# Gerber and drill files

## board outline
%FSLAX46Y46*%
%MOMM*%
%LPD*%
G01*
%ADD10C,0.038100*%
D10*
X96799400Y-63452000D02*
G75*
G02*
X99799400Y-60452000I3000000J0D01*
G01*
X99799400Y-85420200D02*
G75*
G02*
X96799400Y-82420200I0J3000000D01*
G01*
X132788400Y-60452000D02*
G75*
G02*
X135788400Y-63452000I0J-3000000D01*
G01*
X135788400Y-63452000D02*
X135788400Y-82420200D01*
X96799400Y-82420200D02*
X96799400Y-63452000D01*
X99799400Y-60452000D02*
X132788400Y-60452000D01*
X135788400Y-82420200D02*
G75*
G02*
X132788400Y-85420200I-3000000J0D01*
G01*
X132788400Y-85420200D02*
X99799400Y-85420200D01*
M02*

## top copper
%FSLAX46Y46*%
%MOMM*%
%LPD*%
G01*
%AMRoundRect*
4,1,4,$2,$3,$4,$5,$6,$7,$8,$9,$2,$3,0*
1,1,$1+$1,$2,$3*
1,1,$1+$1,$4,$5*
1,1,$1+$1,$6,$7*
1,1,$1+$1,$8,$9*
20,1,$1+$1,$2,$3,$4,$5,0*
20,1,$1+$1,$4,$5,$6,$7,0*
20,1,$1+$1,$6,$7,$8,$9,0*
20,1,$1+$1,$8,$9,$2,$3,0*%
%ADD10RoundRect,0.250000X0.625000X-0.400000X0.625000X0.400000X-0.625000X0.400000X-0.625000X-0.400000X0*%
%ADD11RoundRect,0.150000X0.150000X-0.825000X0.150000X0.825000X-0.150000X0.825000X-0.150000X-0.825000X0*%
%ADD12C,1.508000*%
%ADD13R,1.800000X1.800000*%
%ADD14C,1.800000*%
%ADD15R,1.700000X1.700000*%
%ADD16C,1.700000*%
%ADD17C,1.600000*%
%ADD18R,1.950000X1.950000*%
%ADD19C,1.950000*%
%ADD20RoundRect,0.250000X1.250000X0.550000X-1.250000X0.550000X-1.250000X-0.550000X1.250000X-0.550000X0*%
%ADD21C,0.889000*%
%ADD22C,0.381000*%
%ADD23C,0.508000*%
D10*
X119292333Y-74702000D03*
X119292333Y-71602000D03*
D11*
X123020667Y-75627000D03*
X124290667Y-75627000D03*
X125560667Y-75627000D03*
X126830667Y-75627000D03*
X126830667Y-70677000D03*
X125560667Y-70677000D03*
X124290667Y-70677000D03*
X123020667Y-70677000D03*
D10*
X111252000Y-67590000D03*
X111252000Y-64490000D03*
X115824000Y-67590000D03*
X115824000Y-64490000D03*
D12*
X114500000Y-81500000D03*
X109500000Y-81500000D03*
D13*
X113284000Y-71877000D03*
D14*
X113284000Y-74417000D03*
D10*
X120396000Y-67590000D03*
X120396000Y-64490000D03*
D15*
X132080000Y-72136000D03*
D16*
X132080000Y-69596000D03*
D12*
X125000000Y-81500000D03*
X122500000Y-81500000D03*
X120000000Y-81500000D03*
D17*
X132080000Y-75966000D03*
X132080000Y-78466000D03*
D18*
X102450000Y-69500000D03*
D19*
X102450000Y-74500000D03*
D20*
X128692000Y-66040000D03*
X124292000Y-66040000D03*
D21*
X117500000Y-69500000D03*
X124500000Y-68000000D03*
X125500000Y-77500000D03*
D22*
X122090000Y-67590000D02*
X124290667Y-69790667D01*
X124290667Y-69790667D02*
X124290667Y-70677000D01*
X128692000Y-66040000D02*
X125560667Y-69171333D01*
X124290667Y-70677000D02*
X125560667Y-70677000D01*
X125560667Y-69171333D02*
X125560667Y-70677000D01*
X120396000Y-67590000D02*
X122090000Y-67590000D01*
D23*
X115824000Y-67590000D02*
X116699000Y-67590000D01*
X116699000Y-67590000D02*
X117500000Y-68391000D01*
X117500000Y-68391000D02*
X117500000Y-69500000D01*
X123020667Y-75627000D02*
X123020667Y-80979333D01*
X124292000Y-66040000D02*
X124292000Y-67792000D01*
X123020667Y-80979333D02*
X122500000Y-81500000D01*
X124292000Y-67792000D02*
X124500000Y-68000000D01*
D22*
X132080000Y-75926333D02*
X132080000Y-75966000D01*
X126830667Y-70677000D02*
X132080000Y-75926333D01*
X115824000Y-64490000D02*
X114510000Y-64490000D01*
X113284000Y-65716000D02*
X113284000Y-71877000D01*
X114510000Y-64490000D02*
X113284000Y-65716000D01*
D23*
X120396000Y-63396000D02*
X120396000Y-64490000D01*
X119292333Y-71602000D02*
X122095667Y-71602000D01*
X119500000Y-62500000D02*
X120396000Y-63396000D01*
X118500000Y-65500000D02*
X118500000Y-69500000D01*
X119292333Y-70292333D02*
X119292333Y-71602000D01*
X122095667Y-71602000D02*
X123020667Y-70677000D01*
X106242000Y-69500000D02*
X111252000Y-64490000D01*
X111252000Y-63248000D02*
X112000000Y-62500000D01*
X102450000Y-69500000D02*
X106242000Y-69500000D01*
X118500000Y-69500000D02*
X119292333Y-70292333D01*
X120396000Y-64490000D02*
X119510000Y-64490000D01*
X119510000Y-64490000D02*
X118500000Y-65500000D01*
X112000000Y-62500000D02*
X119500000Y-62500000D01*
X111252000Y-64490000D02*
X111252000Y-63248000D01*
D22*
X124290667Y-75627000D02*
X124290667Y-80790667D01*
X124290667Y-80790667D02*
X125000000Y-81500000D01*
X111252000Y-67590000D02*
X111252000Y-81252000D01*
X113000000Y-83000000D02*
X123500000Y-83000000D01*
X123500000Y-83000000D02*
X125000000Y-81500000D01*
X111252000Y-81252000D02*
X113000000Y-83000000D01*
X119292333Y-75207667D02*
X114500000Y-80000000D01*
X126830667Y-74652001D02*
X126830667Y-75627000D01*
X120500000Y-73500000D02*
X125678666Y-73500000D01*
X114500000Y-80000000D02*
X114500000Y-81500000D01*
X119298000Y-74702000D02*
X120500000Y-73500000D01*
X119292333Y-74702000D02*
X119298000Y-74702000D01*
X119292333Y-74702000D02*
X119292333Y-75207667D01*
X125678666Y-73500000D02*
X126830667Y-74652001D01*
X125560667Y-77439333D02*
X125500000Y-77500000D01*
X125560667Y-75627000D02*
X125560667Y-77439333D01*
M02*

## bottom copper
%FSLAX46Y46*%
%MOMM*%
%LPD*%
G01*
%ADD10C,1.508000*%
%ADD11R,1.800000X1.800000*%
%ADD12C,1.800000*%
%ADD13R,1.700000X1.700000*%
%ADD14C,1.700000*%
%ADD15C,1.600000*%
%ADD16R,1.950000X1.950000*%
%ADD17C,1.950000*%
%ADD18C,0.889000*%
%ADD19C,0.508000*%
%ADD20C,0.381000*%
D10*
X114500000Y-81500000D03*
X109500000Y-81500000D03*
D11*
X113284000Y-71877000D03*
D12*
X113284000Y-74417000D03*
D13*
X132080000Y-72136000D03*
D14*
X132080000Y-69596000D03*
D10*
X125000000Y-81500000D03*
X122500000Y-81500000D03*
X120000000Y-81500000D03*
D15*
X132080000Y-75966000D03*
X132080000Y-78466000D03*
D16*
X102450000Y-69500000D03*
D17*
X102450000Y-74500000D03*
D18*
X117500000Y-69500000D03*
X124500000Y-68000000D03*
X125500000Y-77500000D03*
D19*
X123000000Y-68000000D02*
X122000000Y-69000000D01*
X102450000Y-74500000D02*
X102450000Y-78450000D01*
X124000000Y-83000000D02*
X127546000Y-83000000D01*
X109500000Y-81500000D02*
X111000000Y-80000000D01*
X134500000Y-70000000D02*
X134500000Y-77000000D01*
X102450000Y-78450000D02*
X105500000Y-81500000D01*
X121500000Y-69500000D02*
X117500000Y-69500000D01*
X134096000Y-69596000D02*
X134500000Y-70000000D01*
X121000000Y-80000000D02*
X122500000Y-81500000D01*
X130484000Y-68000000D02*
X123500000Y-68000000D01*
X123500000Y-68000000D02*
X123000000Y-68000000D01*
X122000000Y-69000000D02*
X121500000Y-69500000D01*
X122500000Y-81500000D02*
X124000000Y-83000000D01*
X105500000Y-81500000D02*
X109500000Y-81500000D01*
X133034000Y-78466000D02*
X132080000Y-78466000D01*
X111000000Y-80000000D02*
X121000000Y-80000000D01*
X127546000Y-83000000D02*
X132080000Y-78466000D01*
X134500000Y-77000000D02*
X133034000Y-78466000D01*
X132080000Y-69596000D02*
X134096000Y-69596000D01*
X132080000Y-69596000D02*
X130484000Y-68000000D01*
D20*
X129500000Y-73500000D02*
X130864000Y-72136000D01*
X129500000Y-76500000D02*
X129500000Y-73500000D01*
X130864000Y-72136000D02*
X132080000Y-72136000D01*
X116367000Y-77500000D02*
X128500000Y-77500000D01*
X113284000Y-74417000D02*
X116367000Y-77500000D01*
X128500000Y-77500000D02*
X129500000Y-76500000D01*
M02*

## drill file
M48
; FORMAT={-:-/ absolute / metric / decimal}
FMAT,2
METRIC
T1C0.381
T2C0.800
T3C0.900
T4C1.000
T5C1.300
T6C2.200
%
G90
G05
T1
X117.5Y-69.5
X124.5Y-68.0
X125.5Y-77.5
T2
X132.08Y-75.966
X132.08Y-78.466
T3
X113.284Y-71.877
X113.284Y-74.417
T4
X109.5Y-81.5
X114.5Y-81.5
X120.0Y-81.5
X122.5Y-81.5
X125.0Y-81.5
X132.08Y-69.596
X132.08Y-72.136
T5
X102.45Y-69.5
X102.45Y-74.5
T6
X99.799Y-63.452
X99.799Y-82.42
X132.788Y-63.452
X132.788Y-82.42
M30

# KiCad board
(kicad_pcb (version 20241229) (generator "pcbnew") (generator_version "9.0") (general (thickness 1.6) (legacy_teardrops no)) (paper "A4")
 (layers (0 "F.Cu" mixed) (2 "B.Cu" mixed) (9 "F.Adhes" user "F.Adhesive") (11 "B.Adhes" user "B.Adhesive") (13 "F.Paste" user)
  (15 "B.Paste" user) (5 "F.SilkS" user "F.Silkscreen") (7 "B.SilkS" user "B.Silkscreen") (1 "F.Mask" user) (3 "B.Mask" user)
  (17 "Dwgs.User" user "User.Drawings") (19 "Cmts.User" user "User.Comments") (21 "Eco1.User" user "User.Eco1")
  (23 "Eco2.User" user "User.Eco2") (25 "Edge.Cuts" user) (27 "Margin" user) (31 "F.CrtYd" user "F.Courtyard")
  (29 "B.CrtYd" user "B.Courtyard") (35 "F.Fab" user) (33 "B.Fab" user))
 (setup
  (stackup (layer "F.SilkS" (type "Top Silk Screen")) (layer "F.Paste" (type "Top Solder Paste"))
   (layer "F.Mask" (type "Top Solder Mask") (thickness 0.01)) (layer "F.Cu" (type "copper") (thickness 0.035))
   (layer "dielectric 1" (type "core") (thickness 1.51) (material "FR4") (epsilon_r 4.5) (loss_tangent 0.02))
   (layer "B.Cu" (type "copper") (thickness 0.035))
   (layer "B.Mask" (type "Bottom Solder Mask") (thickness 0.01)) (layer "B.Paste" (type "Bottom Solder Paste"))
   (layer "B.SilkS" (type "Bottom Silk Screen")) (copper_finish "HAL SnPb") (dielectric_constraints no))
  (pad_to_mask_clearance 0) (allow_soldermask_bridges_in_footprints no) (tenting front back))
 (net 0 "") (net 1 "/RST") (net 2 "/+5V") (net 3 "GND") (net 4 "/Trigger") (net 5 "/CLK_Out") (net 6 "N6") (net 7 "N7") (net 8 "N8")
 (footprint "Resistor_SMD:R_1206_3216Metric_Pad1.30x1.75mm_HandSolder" (layer "F.Cu") (at 119.292333 73.152 90)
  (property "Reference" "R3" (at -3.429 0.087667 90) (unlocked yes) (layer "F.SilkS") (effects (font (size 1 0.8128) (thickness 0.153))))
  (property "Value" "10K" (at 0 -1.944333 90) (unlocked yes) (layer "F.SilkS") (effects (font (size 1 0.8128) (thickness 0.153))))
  (pad "1" smd roundrect (at -1.55 0 90) (size 1.3 1.75) (layers "F.Cu" "F.Mask" "F.Paste") (roundrect_rratio 0.192308) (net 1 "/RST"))
  (pad "2" smd roundrect (at 1.55 0 90) (size 1.3 1.75) (layers "F.Cu" "F.Mask" "F.Paste") (roundrect_rratio 0.192308) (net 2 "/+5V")))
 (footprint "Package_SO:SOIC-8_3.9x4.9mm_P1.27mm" (layer "F.Cu") (at 124.925667 73.152 90)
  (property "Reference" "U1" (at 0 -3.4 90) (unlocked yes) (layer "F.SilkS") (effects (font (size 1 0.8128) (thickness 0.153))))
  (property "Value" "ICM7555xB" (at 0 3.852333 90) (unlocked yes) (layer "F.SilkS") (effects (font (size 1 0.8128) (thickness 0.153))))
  (pad "1" smd roundrect (at -2.475 -1.905 90) (size 1.95 0.6) (layers "F.Cu" "F.Mask" "F.Paste") (roundrect_rratio 0.25) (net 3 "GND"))
  (pad "2" smd roundrect (at -2.475 -0.635 90) (size 1.95 0.6) (layers "F.Cu" "F.Mask" "F.Paste") (roundrect_rratio 0.25) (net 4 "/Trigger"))
  (pad "3" smd roundrect (at -2.475 0.635 90) (size 1.95 0.6) (layers "F.Cu" "F.Mask" "F.Paste") (roundrect_rratio 0.25) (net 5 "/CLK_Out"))
  (pad "4" smd roundrect (at -2.475 1.905 90) (size 1.95 0.6) (layers "F.Cu" "F.Mask" "F.Paste") (roundrect_rratio 0.25) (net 1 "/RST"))
  (pad "5" smd roundrect (at 2.475 1.905 90) (size 1.95 0.6) (layers "F.Cu" "F.Mask" "F.Paste") (roundrect_rratio 0.25) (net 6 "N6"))
  (pad "6" smd roundrect (at 2.475 0.635 90) (size 1.95 0.6) (layers "F.Cu" "F.Mask" "F.Paste") (roundrect_rratio 0.25) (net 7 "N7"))
  (pad "7" smd roundrect (at 2.475 -0.635 90) (size 1.95 0.6) (layers "F.Cu" "F.Mask" "F.Paste") (roundrect_rratio 0.25) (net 7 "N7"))
  (pad "8" smd roundrect (at 2.475 -1.905 90) (size 1.95 0.6) (layers "F.Cu" "F.Mask" "F.Paste") (roundrect_rratio 0.25) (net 2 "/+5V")))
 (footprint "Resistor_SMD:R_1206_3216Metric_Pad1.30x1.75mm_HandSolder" (layer "F.Cu") (at 111.252 66.04 90)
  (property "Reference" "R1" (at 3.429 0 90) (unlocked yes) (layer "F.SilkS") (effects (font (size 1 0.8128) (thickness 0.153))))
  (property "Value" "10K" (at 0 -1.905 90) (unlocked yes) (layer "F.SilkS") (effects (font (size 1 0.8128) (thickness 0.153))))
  (pad "1" smd roundrect (at -1.55 0 90) (size 1.3 1.75) (layers "F.Cu" "F.Mask" "F.Paste") (roundrect_rratio 0.192308) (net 4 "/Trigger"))
  (pad "2" smd roundrect (at 1.55 0 90) (size 1.3 1.75) (layers "F.Cu" "F.Mask" "F.Paste") (roundrect_rratio 0.192308) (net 2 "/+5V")))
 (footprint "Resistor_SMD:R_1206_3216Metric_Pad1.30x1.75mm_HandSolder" (layer "F.Cu") (at 115.824 66.04 90)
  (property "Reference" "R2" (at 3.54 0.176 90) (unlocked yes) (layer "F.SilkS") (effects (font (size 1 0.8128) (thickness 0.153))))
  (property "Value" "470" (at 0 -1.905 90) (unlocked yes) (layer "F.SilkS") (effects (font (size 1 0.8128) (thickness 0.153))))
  (pad "1" smd roundrect (at -1.55 0 90) (size 1.3 1.75) (layers "F.Cu" "F.Mask" "F.Paste") (roundrect_rratio 0.192308) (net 3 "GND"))
  (pad "2" smd roundrect (at 1.55 0 90) (size 1.3 1.75) (layers "F.Cu" "F.Mask" "F.Paste") (roundrect_rratio 0.192308) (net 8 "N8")))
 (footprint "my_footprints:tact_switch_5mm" (layer "F.Cu") (at 112 81.5 180)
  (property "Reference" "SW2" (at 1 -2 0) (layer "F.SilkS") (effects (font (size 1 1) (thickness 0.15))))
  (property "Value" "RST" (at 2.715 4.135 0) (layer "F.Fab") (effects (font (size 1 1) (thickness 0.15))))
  (pad "1" thru_hole circle (at -2.5 0 180) (size 1.508 1.508) (drill 1) (layers "*.Cu" "*.Mask") (remove_unused_layers no) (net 1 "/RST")
   (solder_mask_margin 0.102))
  (pad "2" thru_hole circle (at 2.5 0 180) (size 1.508 1.508) (drill 1) (layers "*.Cu" "*.Mask") (remove_unused_layers no) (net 3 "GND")
   (solder_mask_margin 0.102)))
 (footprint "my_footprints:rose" (layer "F.Cu") (at 106 63.5 90)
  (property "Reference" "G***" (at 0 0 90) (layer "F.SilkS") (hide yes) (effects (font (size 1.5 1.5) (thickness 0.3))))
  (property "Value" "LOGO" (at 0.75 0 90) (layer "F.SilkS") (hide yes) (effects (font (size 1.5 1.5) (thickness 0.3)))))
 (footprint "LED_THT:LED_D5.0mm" (layer "F.Cu") (at 113.284 71.877 -90)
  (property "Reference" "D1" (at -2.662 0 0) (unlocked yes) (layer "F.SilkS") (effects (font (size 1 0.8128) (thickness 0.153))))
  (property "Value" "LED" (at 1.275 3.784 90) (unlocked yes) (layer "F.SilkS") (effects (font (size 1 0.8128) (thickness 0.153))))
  (pad "1" thru_hole rect (at 0 0 270) (size 1.8 1.8) (drill 0.9) (layers "*.Cu" "*.Mask") (remove_unused_layers no) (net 8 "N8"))
  (pad "2" thru_hole circle (at 2.54 0 270) (size 1.8 1.8) (drill 0.9) (layers "*.Cu" "*.Mask") (remove_unused_layers no) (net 5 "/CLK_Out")))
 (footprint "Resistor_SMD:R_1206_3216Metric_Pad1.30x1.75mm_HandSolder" (layer "F.Cu") (at 120.396 66.04 90)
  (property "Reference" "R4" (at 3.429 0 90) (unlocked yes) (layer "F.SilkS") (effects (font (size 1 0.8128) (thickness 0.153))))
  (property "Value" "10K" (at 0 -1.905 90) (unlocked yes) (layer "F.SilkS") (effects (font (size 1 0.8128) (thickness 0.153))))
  (pad "1" smd roundrect (at -1.55 0 90) (size 1.3 1.75) (layers "F.Cu" "F.Mask" "F.Paste") (roundrect_rratio 0.192308) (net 7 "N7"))
  (pad "2" smd roundrect (at 1.55 0 90) (size 1.3 1.75) (layers "F.Cu" "F.Mask" "F.Paste") (roundrect_rratio 0.192308) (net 2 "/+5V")))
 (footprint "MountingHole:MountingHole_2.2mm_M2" (layer "F.Cu") (at 99.7994 63.452)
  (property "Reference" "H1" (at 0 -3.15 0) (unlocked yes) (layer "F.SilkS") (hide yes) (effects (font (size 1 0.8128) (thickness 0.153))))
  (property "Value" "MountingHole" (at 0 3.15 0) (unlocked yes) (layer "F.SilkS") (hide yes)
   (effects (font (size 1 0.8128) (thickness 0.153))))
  (pad "" np_thru_hole circle (at 0 0) (size 2.2 2.2) (drill 2.2) (layers "*.Cu" "*.Mask")))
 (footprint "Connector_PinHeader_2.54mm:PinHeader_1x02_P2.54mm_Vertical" (layer "F.Cu") (at 132.08 72.136 180)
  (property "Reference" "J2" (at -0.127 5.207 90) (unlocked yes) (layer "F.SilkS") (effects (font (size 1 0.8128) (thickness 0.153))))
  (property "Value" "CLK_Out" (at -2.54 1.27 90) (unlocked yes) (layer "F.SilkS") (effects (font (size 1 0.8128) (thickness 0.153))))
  (pad "1" thru_hole rect (at 0 0 180) (size 1.7 1.7) (drill 1) (layers "*.Cu" "*.Mask") (remove_unused_layers no) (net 5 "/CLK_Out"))
  (pad "2" thru_hole circle (at 0 2.54 180) (size 1.7 1.7) (drill 1) (layers "*.Cu" "*.Mask") (remove_unused_layers no) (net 3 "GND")))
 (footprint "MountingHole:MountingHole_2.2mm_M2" (layer "F.Cu") (at 132.7884 82.4202)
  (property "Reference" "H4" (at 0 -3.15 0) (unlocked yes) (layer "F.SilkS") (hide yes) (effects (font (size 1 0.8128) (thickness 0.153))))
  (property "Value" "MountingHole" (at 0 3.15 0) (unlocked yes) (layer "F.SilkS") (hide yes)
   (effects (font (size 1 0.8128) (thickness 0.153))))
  (pad "" np_thru_hole circle (at 0 0) (size 2.2 2.2) (drill 2.2) (layers "*.Cu" "*.Mask")))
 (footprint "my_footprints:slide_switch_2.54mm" (layer "F.Cu") (at 122.5 81.5 180)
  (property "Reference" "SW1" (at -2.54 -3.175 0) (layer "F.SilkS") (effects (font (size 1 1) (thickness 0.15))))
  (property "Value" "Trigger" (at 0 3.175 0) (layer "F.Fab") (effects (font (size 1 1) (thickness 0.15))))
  (pad "1" thru_hole circle (at -2.5 0 180) (size 1.508 1.508) (drill 1) (layers "*.Cu" "*.Mask") (remove_unused_layers no)
   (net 4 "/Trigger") (solder_mask_margin 0.102))
  (pad "2" thru_hole circle (at 0 0 180) (size 1.508 1.508) (drill 1) (layers "*.Cu" "*.Mask") (remove_unused_layers no) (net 3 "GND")
   (solder_mask_margin 0.102))
  (pad "3" thru_hole circle (at 2.5 0 180) (size 1.508 1.508) (drill 1) (layers "*.Cu" "*.Mask") (remove_unused_layers no)
   (solder_mask_margin 0.102)))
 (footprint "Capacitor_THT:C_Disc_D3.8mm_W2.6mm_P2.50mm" (layer "F.Cu") (at 132.08 75.966 -90)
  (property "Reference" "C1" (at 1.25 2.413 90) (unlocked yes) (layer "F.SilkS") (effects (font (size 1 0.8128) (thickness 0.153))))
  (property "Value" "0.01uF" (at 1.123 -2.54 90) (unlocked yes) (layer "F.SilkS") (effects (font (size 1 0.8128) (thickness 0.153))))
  (pad "1" thru_hole circle (at 0 0 270) (size 1.6 1.6) (drill 0.8) (layers "*.Cu" "*.Mask") (remove_unused_layers no) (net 6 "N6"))
  (pad "2" thru_hole circle (at 2.5 0 270) (size 1.6 1.6) (drill 0.8) (layers "*.Cu" "*.Mask") (remove_unused_layers no) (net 3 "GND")))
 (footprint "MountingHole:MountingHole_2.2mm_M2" (layer "F.Cu") (at 132.7884 63.452)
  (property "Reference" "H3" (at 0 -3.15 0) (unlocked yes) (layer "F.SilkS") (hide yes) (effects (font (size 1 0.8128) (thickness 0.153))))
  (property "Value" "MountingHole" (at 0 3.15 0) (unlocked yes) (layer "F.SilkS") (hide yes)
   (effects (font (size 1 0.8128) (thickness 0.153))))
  (pad "" np_thru_hole circle (at 0 0) (size 2.2 2.2) (drill 2.2) (layers "*.Cu" "*.Mask")))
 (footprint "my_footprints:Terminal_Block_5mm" (layer "F.Cu") (at 102.45 72 -90)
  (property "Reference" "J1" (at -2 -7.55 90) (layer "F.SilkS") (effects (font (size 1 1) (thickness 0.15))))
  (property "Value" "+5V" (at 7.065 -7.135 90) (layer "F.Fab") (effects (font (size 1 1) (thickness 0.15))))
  (pad "1" thru_hole rect (at -2.5 0 270) (size 1.95 1.95) (drill 1.3) (layers "*.Cu" "*.Mask") (remove_unused_layers no) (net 2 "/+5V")
   (solder_mask_margin 0.102))
  (pad "2" thru_hole circle (at 2.5 0 270) (size 1.95 1.95) (drill 1.3) (layers "*.Cu" "*.Mask") (remove_unused_layers no) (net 3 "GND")
   (solder_mask_margin 0.102)))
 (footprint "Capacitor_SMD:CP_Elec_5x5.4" (layer "F.Cu") (at 126.492 66.04 180)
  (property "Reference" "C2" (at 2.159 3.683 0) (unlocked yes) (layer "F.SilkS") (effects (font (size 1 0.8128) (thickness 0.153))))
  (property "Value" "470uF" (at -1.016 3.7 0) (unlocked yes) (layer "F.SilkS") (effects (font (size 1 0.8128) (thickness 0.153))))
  (pad "1" smd roundrect (at -2.2 0 180) (size 3 1.6) (layers "F.Cu" "F.Mask" "F.Paste") (roundrect_rratio 0.15625) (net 7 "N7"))
  (pad "2" smd roundrect (at 2.2 0 180) (size 3 1.6) (layers "F.Cu" "F.Mask" "F.Paste") (roundrect_rratio 0.15625) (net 3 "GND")))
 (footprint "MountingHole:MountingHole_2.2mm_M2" (layer "F.Cu") (at 99.7994 82.4202)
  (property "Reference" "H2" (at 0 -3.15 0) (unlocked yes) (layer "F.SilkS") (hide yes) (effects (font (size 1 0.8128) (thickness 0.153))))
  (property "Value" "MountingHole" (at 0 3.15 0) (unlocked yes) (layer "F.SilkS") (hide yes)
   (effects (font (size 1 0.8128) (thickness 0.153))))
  (pad "" np_thru_hole circle (at 0 0) (size 2.2 2.2) (drill 2.2) (layers "*.Cu" "*.Mask")))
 (gr_arc (start 96.7994 63.452) (mid 97.67808 61.33068) (end 99.7994 60.452) (stroke (width 0.0381) (type default)) (layer "Edge.Cuts"))
 (gr_arc (start 99.7994 85.4202) (mid 97.67808 84.54152) (end 96.7994 82.4202) (stroke (width 0.0381) (type default)) (layer "Edge.Cuts"))
 (gr_arc (start 132.7884 60.452) (mid 134.90972 61.33068) (end 135.7884 63.452) (stroke (width 0.0381) (type default)) (layer "Edge.Cuts"))
 (gr_line (start 135.7884 63.452) (end 135.7884 82.4202) (stroke (width 0.0381) (type default)) (layer "Edge.Cuts"))
 (gr_line (start 96.7994 82.4202) (end 96.7994 63.452) (stroke (width 0.0381) (type default)) (layer "Edge.Cuts"))
 (gr_line (start 99.7994 60.452) (end 132.7884 60.452) (stroke (width 0.0381) (type default)) (layer "Edge.Cuts"))
 (gr_arc (start 135.7884 82.4202) (mid 134.90972 84.54152) (end 132.7884 85.4202) (stroke (width 0.0381) (type default)) (layer "Edge.Cuts"))
 (gr_line (start 132.7884 85.4202) (end 99.7994 85.4202) (stroke (width 0.0381) (type default)) (layer "Edge.Cuts"))
 (segment (start 122.09 67.59) (end 124.290667 69.790667) (width 0.381) (layer "F.Cu") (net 7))
 (segment (start 124.290667 69.790667) (end 124.290667 70.677) (width 0.381) (layer "F.Cu") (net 7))
 (segment (start 128.692 66.04) (end 125.560667 69.171333) (width 0.381) (layer "F.Cu") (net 7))
 (segment (start 124.290667 70.677) (end 125.560667 70.677) (width 0.381) (layer "F.Cu") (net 7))
 (segment (start 125.560667 69.171333) (end 125.560667 70.677) (width 0.381) (layer "F.Cu") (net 7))
 (segment (start 120.396 67.59) (end 122.09 67.59) (width 0.381) (layer "F.Cu") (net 7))
 (segment (start 115.824 67.59) (end 116.699 67.59) (width 0.508) (layer "F.Cu") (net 3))
 (segment (start 116.699 67.59) (end 117.5 68.391) (width 0.508) (layer "F.Cu") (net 3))
 (segment (start 117.5 68.391) (end 117.5 69.5) (width 0.508) (layer "F.Cu") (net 3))
 (segment (start 123.020667 75.627) (end 123.020667 80.979333) (width 0.508) (layer "F.Cu") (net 3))
 (segment (start 124.292 66.04) (end 124.292 67.792) (width 0.508) (layer "F.Cu") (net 3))
 (segment (start 123.020667 80.979333) (end 122.5 81.5) (width 0.508) (layer "F.Cu") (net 3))
 (segment (start 124.292 67.792) (end 124.5 68) (width 0.508) (layer "F.Cu") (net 3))
 (via (at 117.5 69.5) (size 0.889) (drill 0.381) (layers "F.Cu" "B.Cu") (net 3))
 (via (at 124.5 68) (size 0.889) (drill 0.381) (layers "F.Cu" "B.Cu") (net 3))
 (segment (start 123 68) (end 122 69) (width 0.508) (layer "B.Cu") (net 3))
 (segment (start 102.45 74.5) (end 102.45 78.45) (width 0.508) (layer "B.Cu") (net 3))
 (segment (start 124 83) (end 127.546 83) (width 0.508) (layer "B.Cu") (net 3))
 (segment (start 109.5 81.5) (end 111 80) (width 0.508) (layer "B.Cu") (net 3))
 (segment (start 134.5 70) (end 134.5 77) (width 0.508) (layer "B.Cu") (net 3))
 (segment (start 102.45 78.45) (end 105.5 81.5) (width 0.508) (layer "B.Cu") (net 3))
 (segment (start 121.5 69.5) (end 117.5 69.5) (width 0.508) (layer "B.Cu") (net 3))
 (segment (start 134.096 69.596) (end 134.5 70) (width 0.508) (layer "B.Cu") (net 3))
 (segment (start 121 80) (end 122.5 81.5) (width 0.508) (layer "B.Cu") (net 3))
 (segment (start 130.484 68) (end 123.5 68) (width 0.508) (layer "B.Cu") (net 3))
 (segment (start 123.5 68) (end 123 68) (width 0.508) (layer "B.Cu") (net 3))
 (segment (start 122 69) (end 121.5 69.5) (width 0.508) (layer "B.Cu") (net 3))
 (segment (start 122.5 81.5) (end 124 83) (width 0.508) (layer "B.Cu") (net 3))
 (segment (start 105.5 81.5) (end 109.5 81.5) (width 0.508) (layer "B.Cu") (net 3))
 (segment (start 133.034 78.466) (end 132.08 78.466) (width 0.508) (layer "B.Cu") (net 3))
 (segment (start 111 80) (end 121 80) (width 0.508) (layer "B.Cu") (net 3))
 (segment (start 127.546 83) (end 132.08 78.466) (width 0.508) (layer "B.Cu") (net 3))
 (segment (start 134.5 77) (end 133.034 78.466) (width 0.508) (layer "B.Cu") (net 3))
 (segment (start 132.08 69.596) (end 134.096 69.596) (width 0.508) (layer "B.Cu") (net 3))
 (segment (start 132.08 69.596) (end 130.484 68) (width 0.508) (layer "B.Cu") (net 3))
 (segment (start 132.08 75.926333) (end 132.08 75.966) (width 0.381) (layer "F.Cu") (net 6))
 (segment (start 126.830667 70.677) (end 132.08 75.926333) (width 0.381) (layer "F.Cu") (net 6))
 (segment (start 115.824 64.49) (end 114.51 64.49) (width 0.381) (layer "F.Cu") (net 8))
 (segment (start 113.284 65.716) (end 113.284 71.877) (width 0.381) (layer "F.Cu") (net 8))
 (segment (start 114.51 64.49) (end 113.284 65.716) (width 0.381) (layer "F.Cu") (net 8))
 (segment (start 120.396 63.396) (end 120.396 64.49) (width 0.508) (layer "F.Cu") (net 2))
 (segment (start 119.292333 71.602) (end 122.095667 71.602) (width 0.508) (layer "F.Cu") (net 2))
 (segment (start 119.5 62.5) (end 120.396 63.396) (width 0.508) (layer "F.Cu") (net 2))
 (segment (start 118.5 65.5) (end 118.5 69.5) (width 0.508) (layer "F.Cu") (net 2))
 (segment (start 119.292333 70.292333) (end 119.292333 71.602) (width 0.508) (layer "F.Cu") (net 2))
 (segment (start 122.095667 71.602) (end 123.020667 70.677) (width 0.508) (layer "F.Cu") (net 2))
 (segment (start 106.242 69.5) (end 111.252 64.49) (width 0.508) (layer "F.Cu") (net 2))
 (segment (start 111.252 63.248) (end 112 62.5) (width 0.508) (layer "F.Cu") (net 2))
 (segment (start 102.45 69.5) (end 106.242 69.5) (width 0.508) (layer "F.Cu") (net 2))
 (segment (start 118.5 69.5) (end 119.292333 70.292333) (width 0.508) (layer "F.Cu") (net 2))
 (segment (start 120.396 64.49) (end 119.51 64.49) (width 0.508) (layer "F.Cu") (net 2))
 (segment (start 119.51 64.49) (end 118.5 65.5) (width 0.508) (layer "F.Cu") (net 2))
 (segment (start 112 62.5) (end 119.5 62.5) (width 0.508) (layer "F.Cu") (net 2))
 (segment (start 111.252 64.49) (end 111.252 63.248) (width 0.508) (layer "F.Cu") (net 2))
 (segment (start 124.290667 75.627) (end 124.290667 80.790667) (width 0.381) (layer "F.Cu") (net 4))
 (segment (start 124.290667 80.790667) (end 125 81.5) (width 0.381) (layer "F.Cu") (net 4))
 (segment (start 111.252 67.59) (end 111.252 81.252) (width 0.381) (layer "F.Cu") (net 4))
 (segment (start 113 83) (end 123.5 83) (width 0.381) (layer "F.Cu") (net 4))
 (segment (start 123.5 83) (end 125 81.5) (width 0.381) (layer "F.Cu") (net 4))
 (segment (start 111.252 81.252) (end 113 83) (width 0.381) (layer "F.Cu") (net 4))
 (segment (start 119.292333 75.207667) (end 114.5 80) (width 0.381) (layer "F.Cu") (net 1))
 (segment (start 126.830667 74.652001) (end 126.830667 75.627) (width 0.381) (layer "F.Cu") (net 1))
 (segment (start 120.5 73.5) (end 125.678666 73.5) (width 0.381) (layer "F.Cu") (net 1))
 (segment (start 114.5 80) (end 114.5 81.5) (width 0.381) (layer "F.Cu") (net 1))
 (segment (start 119.298 74.702) (end 120.5 73.5) (width 0.381) (layer "F.Cu") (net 1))
 (segment (start 119.292333 74.702) (end 119.298 74.702) (width 0.381) (layer "F.Cu") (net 1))
 (segment (start 119.292333 74.702) (end 119.292333 75.207667) (width 0.381) (layer "F.Cu") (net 1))
 (segment (start 125.678666 73.5) (end 126.830667 74.652001) (width 0.381) (layer "F.Cu") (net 1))
 (segment (start 125.560667 77.439333) (end 125.5 77.5) (width 0.381) (layer "F.Cu") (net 5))
 (segment (start 125.560667 75.627) (end 125.560667 77.439333) (width 0.381) (layer "F.Cu") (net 5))
 (via (at 125.5 77.5) (size 0.889) (drill 0.381) (layers "F.Cu" "B.Cu") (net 5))
 (segment (start 129.5 73.5) (end 130.864 72.136) (width 0.381) (layer "B.Cu") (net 5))
 (segment (start 129.5 76.5) (end 129.5 73.5) (width 0.381) (layer "B.Cu") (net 5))
 (segment (start 130.864 72.136) (end 132.08 72.136) (width 0.381) (layer "B.Cu") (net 5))
 (segment (start 116.367 77.5) (end 128.5 77.5) (width 0.381) (layer "B.Cu") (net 5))
 (segment (start 113.284 74.417) (end 116.367 77.5) (width 0.381) (layer "B.Cu") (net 5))
 (segment (start 128.5 77.5) (end 129.5 76.5) (width 0.381) (layer "B.Cu") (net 5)))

